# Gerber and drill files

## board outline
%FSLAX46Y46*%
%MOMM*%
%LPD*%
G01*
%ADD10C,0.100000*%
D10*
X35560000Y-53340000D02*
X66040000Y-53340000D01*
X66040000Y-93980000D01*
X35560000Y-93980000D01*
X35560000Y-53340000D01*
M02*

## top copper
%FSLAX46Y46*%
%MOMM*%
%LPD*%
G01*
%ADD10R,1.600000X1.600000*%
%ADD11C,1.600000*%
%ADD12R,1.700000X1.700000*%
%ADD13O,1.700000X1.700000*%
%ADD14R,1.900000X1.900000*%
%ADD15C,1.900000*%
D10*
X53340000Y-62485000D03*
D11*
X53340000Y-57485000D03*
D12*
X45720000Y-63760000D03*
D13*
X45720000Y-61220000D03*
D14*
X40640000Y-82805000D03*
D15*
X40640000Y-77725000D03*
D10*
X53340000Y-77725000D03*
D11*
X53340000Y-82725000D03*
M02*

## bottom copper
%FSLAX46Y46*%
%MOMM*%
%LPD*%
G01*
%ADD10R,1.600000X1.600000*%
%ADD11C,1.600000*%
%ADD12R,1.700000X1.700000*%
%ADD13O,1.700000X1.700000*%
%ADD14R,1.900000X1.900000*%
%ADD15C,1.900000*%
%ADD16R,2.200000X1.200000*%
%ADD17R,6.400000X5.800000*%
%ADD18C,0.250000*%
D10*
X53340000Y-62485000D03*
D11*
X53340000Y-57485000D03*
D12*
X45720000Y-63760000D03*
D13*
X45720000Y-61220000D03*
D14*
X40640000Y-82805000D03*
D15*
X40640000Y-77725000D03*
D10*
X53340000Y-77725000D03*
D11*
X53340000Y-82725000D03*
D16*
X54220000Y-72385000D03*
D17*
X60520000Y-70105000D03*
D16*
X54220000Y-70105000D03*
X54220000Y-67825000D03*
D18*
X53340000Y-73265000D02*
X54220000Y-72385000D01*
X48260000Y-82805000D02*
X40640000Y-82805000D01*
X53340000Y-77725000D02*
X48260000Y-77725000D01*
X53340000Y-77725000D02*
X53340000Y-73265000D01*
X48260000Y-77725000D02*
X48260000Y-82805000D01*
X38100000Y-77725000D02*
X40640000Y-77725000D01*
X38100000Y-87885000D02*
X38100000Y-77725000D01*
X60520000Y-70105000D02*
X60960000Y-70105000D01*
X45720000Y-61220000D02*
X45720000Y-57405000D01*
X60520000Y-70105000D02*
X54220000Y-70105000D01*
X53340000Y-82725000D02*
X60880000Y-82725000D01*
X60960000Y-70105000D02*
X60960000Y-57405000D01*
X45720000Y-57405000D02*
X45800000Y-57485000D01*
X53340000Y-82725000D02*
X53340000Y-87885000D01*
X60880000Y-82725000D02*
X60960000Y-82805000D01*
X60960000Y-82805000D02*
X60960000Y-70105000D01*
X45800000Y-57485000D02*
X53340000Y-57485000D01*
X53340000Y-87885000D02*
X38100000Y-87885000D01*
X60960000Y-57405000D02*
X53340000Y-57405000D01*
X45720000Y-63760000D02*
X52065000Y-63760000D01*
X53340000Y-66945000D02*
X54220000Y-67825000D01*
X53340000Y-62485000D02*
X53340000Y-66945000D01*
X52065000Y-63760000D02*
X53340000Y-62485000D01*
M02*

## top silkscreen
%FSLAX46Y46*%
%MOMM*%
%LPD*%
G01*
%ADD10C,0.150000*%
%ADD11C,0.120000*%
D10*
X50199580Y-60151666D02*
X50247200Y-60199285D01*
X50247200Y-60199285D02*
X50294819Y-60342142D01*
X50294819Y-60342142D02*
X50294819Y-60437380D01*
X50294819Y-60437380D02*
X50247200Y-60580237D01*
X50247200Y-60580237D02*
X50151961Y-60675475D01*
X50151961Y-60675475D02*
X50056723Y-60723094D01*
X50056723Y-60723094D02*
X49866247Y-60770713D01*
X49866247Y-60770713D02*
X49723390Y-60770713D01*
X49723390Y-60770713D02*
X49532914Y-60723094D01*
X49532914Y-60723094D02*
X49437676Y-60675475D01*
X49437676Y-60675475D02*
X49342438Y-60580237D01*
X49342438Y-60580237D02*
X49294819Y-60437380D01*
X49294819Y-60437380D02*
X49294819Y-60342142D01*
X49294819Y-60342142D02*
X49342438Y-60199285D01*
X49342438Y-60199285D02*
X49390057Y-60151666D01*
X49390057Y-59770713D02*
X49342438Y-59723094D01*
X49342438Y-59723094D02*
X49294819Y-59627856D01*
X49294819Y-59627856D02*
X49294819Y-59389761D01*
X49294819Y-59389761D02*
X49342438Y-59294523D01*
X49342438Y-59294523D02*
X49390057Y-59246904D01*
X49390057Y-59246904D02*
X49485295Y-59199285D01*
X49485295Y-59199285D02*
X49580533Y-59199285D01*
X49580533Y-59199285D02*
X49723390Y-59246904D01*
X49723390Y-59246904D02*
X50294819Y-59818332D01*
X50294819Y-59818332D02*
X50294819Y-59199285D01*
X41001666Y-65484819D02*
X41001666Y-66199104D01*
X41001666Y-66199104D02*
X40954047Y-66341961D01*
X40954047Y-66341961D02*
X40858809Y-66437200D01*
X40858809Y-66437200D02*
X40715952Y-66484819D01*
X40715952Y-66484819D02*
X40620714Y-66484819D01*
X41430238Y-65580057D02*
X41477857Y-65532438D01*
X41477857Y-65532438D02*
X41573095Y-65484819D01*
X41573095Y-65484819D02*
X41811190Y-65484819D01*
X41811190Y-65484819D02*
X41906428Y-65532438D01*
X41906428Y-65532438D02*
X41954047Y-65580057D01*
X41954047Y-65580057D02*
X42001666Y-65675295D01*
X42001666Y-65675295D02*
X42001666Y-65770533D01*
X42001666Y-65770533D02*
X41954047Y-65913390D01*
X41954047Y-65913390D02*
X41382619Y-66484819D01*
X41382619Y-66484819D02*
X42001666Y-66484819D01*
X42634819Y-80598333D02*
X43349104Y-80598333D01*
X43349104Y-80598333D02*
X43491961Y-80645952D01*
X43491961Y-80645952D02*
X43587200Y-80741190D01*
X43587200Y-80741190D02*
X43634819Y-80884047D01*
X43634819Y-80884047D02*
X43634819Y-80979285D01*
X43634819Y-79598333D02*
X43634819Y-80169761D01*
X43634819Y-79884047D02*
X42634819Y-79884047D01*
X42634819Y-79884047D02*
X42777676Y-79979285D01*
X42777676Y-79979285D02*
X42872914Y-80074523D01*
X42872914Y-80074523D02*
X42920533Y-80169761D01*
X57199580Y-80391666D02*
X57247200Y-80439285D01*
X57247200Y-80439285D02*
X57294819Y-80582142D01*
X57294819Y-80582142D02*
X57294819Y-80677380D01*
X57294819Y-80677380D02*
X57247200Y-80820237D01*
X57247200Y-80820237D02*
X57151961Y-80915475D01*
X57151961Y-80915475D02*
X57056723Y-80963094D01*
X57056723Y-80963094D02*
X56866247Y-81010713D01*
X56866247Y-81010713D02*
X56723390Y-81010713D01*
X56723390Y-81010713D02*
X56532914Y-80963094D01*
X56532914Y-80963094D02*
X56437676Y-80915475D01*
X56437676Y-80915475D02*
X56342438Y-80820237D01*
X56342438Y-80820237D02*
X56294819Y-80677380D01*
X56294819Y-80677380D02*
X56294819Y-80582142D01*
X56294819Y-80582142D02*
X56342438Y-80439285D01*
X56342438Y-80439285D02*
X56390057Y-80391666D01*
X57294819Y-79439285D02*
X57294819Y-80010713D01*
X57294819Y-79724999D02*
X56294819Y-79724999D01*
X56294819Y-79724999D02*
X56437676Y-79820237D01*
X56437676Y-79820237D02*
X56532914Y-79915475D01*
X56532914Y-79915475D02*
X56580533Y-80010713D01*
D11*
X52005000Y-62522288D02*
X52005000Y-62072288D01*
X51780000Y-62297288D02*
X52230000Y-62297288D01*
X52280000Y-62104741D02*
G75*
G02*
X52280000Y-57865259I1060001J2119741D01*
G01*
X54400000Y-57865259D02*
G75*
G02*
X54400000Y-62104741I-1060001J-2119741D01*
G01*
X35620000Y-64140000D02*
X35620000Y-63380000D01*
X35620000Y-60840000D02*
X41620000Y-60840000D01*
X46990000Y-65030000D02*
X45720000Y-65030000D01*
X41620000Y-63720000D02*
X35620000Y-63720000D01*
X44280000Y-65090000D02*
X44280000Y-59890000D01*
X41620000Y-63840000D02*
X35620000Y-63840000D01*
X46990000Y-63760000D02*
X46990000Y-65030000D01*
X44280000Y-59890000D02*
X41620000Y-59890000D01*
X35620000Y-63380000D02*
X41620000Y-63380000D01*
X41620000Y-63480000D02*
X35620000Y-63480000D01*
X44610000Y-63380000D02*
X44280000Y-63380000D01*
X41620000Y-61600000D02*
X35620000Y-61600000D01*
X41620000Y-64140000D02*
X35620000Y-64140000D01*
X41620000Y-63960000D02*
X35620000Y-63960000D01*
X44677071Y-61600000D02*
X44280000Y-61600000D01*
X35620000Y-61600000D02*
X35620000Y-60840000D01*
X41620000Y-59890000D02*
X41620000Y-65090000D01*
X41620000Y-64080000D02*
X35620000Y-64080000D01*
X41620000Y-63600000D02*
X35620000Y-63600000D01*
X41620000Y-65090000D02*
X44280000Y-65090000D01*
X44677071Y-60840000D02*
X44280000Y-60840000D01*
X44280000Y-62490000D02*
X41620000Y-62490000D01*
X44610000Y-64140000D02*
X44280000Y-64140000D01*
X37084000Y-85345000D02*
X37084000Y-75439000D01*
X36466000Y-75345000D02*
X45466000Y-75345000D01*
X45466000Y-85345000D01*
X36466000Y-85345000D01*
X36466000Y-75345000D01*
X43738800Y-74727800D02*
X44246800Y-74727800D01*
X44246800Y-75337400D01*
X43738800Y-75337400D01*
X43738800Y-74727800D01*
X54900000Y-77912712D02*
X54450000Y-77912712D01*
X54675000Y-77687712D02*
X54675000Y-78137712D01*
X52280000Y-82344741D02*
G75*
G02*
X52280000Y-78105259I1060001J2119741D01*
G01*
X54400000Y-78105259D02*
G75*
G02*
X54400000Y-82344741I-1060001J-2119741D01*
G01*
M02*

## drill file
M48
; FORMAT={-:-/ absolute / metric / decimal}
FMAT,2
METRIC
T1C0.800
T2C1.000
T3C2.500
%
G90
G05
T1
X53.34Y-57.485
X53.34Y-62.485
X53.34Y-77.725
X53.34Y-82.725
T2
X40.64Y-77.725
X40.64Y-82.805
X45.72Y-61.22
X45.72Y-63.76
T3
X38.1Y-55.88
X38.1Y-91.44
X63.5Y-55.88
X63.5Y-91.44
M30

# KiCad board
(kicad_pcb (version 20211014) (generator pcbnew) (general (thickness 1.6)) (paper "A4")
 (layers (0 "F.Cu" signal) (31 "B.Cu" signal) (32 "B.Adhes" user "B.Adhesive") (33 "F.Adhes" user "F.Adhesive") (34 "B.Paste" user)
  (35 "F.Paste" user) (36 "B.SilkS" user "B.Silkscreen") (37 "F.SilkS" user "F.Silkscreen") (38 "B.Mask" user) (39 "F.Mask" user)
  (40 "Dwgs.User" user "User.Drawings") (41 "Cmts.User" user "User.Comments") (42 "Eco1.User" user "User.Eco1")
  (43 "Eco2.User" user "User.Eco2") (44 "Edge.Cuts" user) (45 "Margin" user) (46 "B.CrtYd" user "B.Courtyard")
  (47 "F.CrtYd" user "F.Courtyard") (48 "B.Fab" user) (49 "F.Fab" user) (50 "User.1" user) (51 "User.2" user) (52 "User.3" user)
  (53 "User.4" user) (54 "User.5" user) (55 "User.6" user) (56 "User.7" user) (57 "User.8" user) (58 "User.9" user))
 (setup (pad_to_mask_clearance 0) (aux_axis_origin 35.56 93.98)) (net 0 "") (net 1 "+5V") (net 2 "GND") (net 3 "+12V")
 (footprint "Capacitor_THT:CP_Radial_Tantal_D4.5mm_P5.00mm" (layer "F.Cu") (at 53.34 62.485 90)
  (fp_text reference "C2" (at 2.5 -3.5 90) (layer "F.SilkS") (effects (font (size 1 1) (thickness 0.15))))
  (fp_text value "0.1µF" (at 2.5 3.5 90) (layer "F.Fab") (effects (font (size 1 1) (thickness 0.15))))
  (fp_line (start -0.037288 -1.335) (end 0.412712 -1.335) (layer "F.SilkS") (width 0.12))
  (fp_line (start 0.187712 -1.56) (end 0.187712 -1.11) (layer "F.SilkS") (width 0.12))
  (fp_arc (start 0.380259 -1.06) (mid 2.5 -2.37) (end 4.619741 -1.06) (layer "F.SilkS") (width 0.12))
  (fp_arc (start 4.619741 1.06) (mid 2.5 2.37) (end 0.380259 1.06) (layer "F.SilkS") (width 0.12))
  (pad "1" thru_hole rect (at 0 0 90) (size 1.6 1.6) (drill 0.8) (layers *.Cu *.Mask) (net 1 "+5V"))
  (pad "2" thru_hole circle (at 5 0 90) (size 1.6 1.6) (drill 0.8) (layers *.Cu *.Mask) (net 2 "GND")))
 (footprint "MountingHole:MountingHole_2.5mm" (layer "F.Cu") (at 63.5 55.88)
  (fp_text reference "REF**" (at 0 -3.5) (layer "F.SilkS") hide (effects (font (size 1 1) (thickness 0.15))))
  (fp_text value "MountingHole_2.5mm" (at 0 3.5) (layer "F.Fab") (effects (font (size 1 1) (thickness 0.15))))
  (pad "" np_thru_hole circle (at 0 0) (size 2.5 2.5) (drill 2.5) (layers *.Cu *.Mask)))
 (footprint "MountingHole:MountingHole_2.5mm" (layer "F.Cu") (at 38.1 55.88)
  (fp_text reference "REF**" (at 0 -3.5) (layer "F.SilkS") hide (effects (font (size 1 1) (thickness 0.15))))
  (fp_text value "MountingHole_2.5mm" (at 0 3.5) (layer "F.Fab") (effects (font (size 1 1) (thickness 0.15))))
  (pad "" np_thru_hole circle (at 0 0) (size 2.5 2.5) (drill 2.5) (layers *.Mask)))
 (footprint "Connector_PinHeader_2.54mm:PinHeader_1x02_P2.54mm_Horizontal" (layer "F.Cu") (at 45.72 63.76 180)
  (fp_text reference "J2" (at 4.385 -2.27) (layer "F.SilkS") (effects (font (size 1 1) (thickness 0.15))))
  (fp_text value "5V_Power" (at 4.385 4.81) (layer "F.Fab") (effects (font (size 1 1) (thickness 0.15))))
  (fp_line (start 10.1 -0.38) (end 10.1 0.38) (layer "F.SilkS") (width 0.12))
  (fp_line (start 10.1 2.92) (end 4.1 2.92) (layer "F.SilkS") (width 0.12))
  (fp_line (start -1.27 -1.27) (end 0 -1.27) (layer "F.SilkS") (width 0.12))
  (fp_line (start 4.1 0.04) (end 10.1 0.04) (layer "F.SilkS") (width 0.12))
  (fp_line (start 1.44 -1.33) (end 1.44 3.87) (layer "F.SilkS") (width 0.12))
  (fp_line (start 4.1 -0.08) (end 10.1 -0.08) (layer "F.SilkS") (width 0.12))
  (fp_line (start -1.27 0) (end -1.27 -1.27) (layer "F.SilkS") (width 0.12))
  (fp_line (start 1.44 3.87) (end 4.1 3.87) (layer "F.SilkS") (width 0.12))
  (fp_line (start 10.1 0.38) (end 4.1 0.38) (layer "F.SilkS") (width 0.12))
  (fp_line (start 4.1 0.28) (end 10.1 0.28) (layer "F.SilkS") (width 0.12))
  (fp_line (start 1.11 0.38) (end 1.44 0.38) (layer "F.SilkS") (width 0.12))
  (fp_line (start 4.1 2.16) (end 10.1 2.16) (layer "F.SilkS") (width 0.12))
  (fp_line (start 4.1 -0.38) (end 10.1 -0.38) (layer "F.SilkS") (width 0.12))
  (fp_line (start 4.1 -0.2) (end 10.1 -0.2) (layer "F.SilkS") (width 0.12))
  (fp_line (start 1.042929 2.16) (end 1.44 2.16) (layer "F.SilkS") (width 0.12))
  (fp_line (start 10.1 2.16) (end 10.1 2.92) (layer "F.SilkS") (width 0.12))
  (fp_line (start 4.1 3.87) (end 4.1 -1.33) (layer "F.SilkS") (width 0.12))
  (fp_line (start 4.1 -0.32) (end 10.1 -0.32) (layer "F.SilkS") (width 0.12))
  (fp_line (start 4.1 0.16) (end 10.1 0.16) (layer "F.SilkS") (width 0.12))
  (fp_line (start 4.1 -1.33) (end 1.44 -1.33) (layer "F.SilkS") (width 0.12))
  (fp_line (start 1.042929 2.92) (end 1.44 2.92) (layer "F.SilkS") (width 0.12))
  (fp_line (start 1.44 1.27) (end 4.1 1.27) (layer "F.SilkS") (width 0.12))
  (fp_line (start 1.11 -0.38) (end 1.44 -0.38) (layer "F.SilkS") (width 0.12))
  (pad "1" thru_hole rect (at 0 0 180) (size 1.7 1.7) (drill 1) (layers *.Cu *.Mask) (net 1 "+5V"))
  (pad "2" thru_hole oval (at 0 2.54 180) (size 1.7 1.7) (drill 1) (layers *.Cu *.Mask) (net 2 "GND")))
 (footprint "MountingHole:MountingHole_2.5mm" (layer "F.Cu") (at 63.5 91.44)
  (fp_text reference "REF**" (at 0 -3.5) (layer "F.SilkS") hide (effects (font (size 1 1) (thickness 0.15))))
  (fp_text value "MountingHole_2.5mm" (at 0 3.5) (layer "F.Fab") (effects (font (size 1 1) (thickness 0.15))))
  (pad "" np_thru_hole circle (at 0 0) (size 2.5 2.5) (drill 2.5) (layers *.Cu *.Mask)))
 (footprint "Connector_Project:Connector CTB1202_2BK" (layer "F.Cu") (at 40.64 82.805 90)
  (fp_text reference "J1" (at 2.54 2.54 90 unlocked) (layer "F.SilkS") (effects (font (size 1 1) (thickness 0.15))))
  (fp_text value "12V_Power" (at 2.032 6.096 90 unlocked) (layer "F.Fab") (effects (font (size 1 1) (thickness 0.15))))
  (fp_line (start -2.54 -3.556) (end 7.366 -3.556) (layer "F.SilkS") (width 0.12))
  (fp_rect (start -2.54 -4.174) (end 7.46 4.826) (layer "F.SilkS") (width 0.12) (fill none))
  (fp_rect (start 7.4676 3.6068) (end 8.0772 3.0988) (layer "F.SilkS") (width 0.12) (fill none))
  (pad "1" thru_hole rect (at 0 0 90) (size 1.9 1.9) (drill 1) (layers *.Cu *.Mask) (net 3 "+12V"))
  (pad "2" thru_hole circle (at 5.08 0 90) (size 1.9 1.9) (drill 1) (layers *.Cu *.Mask) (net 2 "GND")))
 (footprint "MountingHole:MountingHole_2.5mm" (layer "F.Cu") (at 38.1 91.44)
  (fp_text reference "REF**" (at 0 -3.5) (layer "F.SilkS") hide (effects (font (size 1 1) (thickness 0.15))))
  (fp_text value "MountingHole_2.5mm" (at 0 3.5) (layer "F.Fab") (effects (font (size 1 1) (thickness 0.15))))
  (pad "" np_thru_hole circle (at 0 0) (size 2.5 2.5) (drill 2.5) (layers *.Cu *.Mask)))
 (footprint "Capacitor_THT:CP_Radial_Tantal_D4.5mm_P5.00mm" (layer "F.Cu") (at 53.34 77.725 -90)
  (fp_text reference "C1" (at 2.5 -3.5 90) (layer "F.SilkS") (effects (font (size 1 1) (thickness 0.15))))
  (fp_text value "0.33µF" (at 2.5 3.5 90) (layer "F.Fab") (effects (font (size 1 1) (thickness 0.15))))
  (fp_line (start 0.187712 -1.56) (end 0.187712 -1.11) (layer "F.SilkS") (width 0.12))
  (fp_line (start -0.037288 -1.335) (end 0.412712 -1.335) (layer "F.SilkS") (width 0.12))
  (fp_arc (start 4.619741 1.06) (mid 2.5 2.37) (end 0.380259 1.06) (layer "F.SilkS") (width 0.12))
  (fp_arc (start 0.380259 -1.06) (mid 2.5 -2.37) (end 4.619741 -1.06) (layer "F.SilkS") (width 0.12))
  (pad "1" thru_hole rect (at 0 0 270) (size 1.6 1.6) (drill 0.8) (layers *.Cu *.Mask) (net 3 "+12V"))
  (pad "2" thru_hole circle (at 5 0 270) (size 1.6 1.6) (drill 0.8) (layers *.Cu *.Mask) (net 2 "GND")))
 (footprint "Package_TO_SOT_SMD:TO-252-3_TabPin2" (layer "B.Cu") (at 58.42 70.105)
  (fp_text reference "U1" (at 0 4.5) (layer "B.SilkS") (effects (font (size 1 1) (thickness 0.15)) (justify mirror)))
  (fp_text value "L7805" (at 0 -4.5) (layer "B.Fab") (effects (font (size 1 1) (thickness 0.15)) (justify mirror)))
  (pad "" smd rect (at 0.425 1.525) (size 3.05 2.75) (layers "B.Paste"))
  (pad "" smd rect (at 0.425 -1.525) (size 3.05 2.75) (layers "B.Paste"))
  (pad "" smd rect (at 3.775 -1.525) (size 3.05 2.75) (layers "B.Paste"))
  (pad "" smd rect (at 3.775 1.525) (size 3.05 2.75) (layers "B.Paste"))
  (pad "1" smd rect (at -4.2 2.28) (size 2.2 1.2) (layers "B.Cu" "B.Paste" "B.Mask") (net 3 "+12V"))
  (pad "2" smd rect (at 2.1 0) (size 6.4 5.8) (layers "B.Cu" "B.Mask") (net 2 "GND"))
  (pad "2" smd rect (at -4.2 0) (size 2.2 1.2) (layers "B.Cu" "B.Paste" "B.Mask") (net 2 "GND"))
  (pad "3" smd rect (at -4.2 -2.28) (size 2.2 1.2) (layers "B.Cu" "B.Paste" "B.Mask") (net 1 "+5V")))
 (gr_rect (start 35.56 53.34) (end 66.04 93.98) (layer "Edge.Cuts") (width 0.1) (fill none))
 (segment (start 53.34 73.265) (end 54.22 72.385) (width 0.25) (layer "B.Cu") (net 3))
 (segment (start 48.26 82.805) (end 40.64 82.805) (width 0.25) (layer "B.Cu") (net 3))
 (segment (start 53.34 77.725) (end 48.26 77.725) (width 0.25) (layer "B.Cu") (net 3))
 (segment (start 53.34 77.725) (end 53.34 73.265) (width 0.25) (layer "B.Cu") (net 3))
 (segment (start 48.26 77.725) (end 48.26 82.805) (width 0.25) (layer "B.Cu") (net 3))
 (segment (start 38.1 77.725) (end 40.64 77.725) (width 0.25) (layer "B.Cu") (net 2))
 (segment (start 38.1 87.885) (end 38.1 77.725) (width 0.25) (layer "B.Cu") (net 2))
 (segment (start 60.52 70.105) (end 60.96 70.105) (width 0.25) (layer "B.Cu") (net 2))
 (segment (start 45.72 61.22) (end 45.72 57.405) (width 0.25) (layer "B.Cu") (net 2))
 (segment (start 60.52 70.105) (end 54.22 70.105) (width 0.25) (layer "B.Cu") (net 2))
 (segment (start 53.34 82.725) (end 60.88 82.725) (width 0.25) (layer "B.Cu") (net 2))
 (segment (start 60.96 70.105) (end 60.96 57.405) (width 0.25) (layer "B.Cu") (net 2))
 (segment (start 45.72 57.405) (end 45.8 57.485) (width 0.25) (layer "B.Cu") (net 2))
 (segment (start 53.34 82.725) (end 53.34 87.885) (width 0.25) (layer "B.Cu") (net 2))
 (segment (start 60.88 82.725) (end 60.96 82.805) (width 0.25) (layer "B.Cu") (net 2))
 (segment (start 60.96 82.805) (end 60.96 70.105) (width 0.25) (layer "B.Cu") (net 2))
 (segment (start 45.8 57.485) (end 53.34 57.485) (width 0.25) (layer "B.Cu") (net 2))
 (segment (start 53.34 87.885) (end 38.1 87.885) (width 0.25) (layer "B.Cu") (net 2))
 (segment (start 60.96 57.405) (end 53.34 57.405) (width 0.25) (layer "B.Cu") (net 2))
 (segment (start 45.72 63.76) (end 52.065 63.76) (width 0.25) (layer "B.Cu") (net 1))
 (segment (start 53.34 66.945) (end 54.22 67.825) (width 0.25) (layer "B.Cu") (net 1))
 (segment (start 53.34 62.485) (end 53.34 66.945) (width 0.25) (layer "B.Cu") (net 1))
 (segment (start 52.065 63.76) (end 53.34 62.485) (width 0.25) (layer "B.Cu") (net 1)))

